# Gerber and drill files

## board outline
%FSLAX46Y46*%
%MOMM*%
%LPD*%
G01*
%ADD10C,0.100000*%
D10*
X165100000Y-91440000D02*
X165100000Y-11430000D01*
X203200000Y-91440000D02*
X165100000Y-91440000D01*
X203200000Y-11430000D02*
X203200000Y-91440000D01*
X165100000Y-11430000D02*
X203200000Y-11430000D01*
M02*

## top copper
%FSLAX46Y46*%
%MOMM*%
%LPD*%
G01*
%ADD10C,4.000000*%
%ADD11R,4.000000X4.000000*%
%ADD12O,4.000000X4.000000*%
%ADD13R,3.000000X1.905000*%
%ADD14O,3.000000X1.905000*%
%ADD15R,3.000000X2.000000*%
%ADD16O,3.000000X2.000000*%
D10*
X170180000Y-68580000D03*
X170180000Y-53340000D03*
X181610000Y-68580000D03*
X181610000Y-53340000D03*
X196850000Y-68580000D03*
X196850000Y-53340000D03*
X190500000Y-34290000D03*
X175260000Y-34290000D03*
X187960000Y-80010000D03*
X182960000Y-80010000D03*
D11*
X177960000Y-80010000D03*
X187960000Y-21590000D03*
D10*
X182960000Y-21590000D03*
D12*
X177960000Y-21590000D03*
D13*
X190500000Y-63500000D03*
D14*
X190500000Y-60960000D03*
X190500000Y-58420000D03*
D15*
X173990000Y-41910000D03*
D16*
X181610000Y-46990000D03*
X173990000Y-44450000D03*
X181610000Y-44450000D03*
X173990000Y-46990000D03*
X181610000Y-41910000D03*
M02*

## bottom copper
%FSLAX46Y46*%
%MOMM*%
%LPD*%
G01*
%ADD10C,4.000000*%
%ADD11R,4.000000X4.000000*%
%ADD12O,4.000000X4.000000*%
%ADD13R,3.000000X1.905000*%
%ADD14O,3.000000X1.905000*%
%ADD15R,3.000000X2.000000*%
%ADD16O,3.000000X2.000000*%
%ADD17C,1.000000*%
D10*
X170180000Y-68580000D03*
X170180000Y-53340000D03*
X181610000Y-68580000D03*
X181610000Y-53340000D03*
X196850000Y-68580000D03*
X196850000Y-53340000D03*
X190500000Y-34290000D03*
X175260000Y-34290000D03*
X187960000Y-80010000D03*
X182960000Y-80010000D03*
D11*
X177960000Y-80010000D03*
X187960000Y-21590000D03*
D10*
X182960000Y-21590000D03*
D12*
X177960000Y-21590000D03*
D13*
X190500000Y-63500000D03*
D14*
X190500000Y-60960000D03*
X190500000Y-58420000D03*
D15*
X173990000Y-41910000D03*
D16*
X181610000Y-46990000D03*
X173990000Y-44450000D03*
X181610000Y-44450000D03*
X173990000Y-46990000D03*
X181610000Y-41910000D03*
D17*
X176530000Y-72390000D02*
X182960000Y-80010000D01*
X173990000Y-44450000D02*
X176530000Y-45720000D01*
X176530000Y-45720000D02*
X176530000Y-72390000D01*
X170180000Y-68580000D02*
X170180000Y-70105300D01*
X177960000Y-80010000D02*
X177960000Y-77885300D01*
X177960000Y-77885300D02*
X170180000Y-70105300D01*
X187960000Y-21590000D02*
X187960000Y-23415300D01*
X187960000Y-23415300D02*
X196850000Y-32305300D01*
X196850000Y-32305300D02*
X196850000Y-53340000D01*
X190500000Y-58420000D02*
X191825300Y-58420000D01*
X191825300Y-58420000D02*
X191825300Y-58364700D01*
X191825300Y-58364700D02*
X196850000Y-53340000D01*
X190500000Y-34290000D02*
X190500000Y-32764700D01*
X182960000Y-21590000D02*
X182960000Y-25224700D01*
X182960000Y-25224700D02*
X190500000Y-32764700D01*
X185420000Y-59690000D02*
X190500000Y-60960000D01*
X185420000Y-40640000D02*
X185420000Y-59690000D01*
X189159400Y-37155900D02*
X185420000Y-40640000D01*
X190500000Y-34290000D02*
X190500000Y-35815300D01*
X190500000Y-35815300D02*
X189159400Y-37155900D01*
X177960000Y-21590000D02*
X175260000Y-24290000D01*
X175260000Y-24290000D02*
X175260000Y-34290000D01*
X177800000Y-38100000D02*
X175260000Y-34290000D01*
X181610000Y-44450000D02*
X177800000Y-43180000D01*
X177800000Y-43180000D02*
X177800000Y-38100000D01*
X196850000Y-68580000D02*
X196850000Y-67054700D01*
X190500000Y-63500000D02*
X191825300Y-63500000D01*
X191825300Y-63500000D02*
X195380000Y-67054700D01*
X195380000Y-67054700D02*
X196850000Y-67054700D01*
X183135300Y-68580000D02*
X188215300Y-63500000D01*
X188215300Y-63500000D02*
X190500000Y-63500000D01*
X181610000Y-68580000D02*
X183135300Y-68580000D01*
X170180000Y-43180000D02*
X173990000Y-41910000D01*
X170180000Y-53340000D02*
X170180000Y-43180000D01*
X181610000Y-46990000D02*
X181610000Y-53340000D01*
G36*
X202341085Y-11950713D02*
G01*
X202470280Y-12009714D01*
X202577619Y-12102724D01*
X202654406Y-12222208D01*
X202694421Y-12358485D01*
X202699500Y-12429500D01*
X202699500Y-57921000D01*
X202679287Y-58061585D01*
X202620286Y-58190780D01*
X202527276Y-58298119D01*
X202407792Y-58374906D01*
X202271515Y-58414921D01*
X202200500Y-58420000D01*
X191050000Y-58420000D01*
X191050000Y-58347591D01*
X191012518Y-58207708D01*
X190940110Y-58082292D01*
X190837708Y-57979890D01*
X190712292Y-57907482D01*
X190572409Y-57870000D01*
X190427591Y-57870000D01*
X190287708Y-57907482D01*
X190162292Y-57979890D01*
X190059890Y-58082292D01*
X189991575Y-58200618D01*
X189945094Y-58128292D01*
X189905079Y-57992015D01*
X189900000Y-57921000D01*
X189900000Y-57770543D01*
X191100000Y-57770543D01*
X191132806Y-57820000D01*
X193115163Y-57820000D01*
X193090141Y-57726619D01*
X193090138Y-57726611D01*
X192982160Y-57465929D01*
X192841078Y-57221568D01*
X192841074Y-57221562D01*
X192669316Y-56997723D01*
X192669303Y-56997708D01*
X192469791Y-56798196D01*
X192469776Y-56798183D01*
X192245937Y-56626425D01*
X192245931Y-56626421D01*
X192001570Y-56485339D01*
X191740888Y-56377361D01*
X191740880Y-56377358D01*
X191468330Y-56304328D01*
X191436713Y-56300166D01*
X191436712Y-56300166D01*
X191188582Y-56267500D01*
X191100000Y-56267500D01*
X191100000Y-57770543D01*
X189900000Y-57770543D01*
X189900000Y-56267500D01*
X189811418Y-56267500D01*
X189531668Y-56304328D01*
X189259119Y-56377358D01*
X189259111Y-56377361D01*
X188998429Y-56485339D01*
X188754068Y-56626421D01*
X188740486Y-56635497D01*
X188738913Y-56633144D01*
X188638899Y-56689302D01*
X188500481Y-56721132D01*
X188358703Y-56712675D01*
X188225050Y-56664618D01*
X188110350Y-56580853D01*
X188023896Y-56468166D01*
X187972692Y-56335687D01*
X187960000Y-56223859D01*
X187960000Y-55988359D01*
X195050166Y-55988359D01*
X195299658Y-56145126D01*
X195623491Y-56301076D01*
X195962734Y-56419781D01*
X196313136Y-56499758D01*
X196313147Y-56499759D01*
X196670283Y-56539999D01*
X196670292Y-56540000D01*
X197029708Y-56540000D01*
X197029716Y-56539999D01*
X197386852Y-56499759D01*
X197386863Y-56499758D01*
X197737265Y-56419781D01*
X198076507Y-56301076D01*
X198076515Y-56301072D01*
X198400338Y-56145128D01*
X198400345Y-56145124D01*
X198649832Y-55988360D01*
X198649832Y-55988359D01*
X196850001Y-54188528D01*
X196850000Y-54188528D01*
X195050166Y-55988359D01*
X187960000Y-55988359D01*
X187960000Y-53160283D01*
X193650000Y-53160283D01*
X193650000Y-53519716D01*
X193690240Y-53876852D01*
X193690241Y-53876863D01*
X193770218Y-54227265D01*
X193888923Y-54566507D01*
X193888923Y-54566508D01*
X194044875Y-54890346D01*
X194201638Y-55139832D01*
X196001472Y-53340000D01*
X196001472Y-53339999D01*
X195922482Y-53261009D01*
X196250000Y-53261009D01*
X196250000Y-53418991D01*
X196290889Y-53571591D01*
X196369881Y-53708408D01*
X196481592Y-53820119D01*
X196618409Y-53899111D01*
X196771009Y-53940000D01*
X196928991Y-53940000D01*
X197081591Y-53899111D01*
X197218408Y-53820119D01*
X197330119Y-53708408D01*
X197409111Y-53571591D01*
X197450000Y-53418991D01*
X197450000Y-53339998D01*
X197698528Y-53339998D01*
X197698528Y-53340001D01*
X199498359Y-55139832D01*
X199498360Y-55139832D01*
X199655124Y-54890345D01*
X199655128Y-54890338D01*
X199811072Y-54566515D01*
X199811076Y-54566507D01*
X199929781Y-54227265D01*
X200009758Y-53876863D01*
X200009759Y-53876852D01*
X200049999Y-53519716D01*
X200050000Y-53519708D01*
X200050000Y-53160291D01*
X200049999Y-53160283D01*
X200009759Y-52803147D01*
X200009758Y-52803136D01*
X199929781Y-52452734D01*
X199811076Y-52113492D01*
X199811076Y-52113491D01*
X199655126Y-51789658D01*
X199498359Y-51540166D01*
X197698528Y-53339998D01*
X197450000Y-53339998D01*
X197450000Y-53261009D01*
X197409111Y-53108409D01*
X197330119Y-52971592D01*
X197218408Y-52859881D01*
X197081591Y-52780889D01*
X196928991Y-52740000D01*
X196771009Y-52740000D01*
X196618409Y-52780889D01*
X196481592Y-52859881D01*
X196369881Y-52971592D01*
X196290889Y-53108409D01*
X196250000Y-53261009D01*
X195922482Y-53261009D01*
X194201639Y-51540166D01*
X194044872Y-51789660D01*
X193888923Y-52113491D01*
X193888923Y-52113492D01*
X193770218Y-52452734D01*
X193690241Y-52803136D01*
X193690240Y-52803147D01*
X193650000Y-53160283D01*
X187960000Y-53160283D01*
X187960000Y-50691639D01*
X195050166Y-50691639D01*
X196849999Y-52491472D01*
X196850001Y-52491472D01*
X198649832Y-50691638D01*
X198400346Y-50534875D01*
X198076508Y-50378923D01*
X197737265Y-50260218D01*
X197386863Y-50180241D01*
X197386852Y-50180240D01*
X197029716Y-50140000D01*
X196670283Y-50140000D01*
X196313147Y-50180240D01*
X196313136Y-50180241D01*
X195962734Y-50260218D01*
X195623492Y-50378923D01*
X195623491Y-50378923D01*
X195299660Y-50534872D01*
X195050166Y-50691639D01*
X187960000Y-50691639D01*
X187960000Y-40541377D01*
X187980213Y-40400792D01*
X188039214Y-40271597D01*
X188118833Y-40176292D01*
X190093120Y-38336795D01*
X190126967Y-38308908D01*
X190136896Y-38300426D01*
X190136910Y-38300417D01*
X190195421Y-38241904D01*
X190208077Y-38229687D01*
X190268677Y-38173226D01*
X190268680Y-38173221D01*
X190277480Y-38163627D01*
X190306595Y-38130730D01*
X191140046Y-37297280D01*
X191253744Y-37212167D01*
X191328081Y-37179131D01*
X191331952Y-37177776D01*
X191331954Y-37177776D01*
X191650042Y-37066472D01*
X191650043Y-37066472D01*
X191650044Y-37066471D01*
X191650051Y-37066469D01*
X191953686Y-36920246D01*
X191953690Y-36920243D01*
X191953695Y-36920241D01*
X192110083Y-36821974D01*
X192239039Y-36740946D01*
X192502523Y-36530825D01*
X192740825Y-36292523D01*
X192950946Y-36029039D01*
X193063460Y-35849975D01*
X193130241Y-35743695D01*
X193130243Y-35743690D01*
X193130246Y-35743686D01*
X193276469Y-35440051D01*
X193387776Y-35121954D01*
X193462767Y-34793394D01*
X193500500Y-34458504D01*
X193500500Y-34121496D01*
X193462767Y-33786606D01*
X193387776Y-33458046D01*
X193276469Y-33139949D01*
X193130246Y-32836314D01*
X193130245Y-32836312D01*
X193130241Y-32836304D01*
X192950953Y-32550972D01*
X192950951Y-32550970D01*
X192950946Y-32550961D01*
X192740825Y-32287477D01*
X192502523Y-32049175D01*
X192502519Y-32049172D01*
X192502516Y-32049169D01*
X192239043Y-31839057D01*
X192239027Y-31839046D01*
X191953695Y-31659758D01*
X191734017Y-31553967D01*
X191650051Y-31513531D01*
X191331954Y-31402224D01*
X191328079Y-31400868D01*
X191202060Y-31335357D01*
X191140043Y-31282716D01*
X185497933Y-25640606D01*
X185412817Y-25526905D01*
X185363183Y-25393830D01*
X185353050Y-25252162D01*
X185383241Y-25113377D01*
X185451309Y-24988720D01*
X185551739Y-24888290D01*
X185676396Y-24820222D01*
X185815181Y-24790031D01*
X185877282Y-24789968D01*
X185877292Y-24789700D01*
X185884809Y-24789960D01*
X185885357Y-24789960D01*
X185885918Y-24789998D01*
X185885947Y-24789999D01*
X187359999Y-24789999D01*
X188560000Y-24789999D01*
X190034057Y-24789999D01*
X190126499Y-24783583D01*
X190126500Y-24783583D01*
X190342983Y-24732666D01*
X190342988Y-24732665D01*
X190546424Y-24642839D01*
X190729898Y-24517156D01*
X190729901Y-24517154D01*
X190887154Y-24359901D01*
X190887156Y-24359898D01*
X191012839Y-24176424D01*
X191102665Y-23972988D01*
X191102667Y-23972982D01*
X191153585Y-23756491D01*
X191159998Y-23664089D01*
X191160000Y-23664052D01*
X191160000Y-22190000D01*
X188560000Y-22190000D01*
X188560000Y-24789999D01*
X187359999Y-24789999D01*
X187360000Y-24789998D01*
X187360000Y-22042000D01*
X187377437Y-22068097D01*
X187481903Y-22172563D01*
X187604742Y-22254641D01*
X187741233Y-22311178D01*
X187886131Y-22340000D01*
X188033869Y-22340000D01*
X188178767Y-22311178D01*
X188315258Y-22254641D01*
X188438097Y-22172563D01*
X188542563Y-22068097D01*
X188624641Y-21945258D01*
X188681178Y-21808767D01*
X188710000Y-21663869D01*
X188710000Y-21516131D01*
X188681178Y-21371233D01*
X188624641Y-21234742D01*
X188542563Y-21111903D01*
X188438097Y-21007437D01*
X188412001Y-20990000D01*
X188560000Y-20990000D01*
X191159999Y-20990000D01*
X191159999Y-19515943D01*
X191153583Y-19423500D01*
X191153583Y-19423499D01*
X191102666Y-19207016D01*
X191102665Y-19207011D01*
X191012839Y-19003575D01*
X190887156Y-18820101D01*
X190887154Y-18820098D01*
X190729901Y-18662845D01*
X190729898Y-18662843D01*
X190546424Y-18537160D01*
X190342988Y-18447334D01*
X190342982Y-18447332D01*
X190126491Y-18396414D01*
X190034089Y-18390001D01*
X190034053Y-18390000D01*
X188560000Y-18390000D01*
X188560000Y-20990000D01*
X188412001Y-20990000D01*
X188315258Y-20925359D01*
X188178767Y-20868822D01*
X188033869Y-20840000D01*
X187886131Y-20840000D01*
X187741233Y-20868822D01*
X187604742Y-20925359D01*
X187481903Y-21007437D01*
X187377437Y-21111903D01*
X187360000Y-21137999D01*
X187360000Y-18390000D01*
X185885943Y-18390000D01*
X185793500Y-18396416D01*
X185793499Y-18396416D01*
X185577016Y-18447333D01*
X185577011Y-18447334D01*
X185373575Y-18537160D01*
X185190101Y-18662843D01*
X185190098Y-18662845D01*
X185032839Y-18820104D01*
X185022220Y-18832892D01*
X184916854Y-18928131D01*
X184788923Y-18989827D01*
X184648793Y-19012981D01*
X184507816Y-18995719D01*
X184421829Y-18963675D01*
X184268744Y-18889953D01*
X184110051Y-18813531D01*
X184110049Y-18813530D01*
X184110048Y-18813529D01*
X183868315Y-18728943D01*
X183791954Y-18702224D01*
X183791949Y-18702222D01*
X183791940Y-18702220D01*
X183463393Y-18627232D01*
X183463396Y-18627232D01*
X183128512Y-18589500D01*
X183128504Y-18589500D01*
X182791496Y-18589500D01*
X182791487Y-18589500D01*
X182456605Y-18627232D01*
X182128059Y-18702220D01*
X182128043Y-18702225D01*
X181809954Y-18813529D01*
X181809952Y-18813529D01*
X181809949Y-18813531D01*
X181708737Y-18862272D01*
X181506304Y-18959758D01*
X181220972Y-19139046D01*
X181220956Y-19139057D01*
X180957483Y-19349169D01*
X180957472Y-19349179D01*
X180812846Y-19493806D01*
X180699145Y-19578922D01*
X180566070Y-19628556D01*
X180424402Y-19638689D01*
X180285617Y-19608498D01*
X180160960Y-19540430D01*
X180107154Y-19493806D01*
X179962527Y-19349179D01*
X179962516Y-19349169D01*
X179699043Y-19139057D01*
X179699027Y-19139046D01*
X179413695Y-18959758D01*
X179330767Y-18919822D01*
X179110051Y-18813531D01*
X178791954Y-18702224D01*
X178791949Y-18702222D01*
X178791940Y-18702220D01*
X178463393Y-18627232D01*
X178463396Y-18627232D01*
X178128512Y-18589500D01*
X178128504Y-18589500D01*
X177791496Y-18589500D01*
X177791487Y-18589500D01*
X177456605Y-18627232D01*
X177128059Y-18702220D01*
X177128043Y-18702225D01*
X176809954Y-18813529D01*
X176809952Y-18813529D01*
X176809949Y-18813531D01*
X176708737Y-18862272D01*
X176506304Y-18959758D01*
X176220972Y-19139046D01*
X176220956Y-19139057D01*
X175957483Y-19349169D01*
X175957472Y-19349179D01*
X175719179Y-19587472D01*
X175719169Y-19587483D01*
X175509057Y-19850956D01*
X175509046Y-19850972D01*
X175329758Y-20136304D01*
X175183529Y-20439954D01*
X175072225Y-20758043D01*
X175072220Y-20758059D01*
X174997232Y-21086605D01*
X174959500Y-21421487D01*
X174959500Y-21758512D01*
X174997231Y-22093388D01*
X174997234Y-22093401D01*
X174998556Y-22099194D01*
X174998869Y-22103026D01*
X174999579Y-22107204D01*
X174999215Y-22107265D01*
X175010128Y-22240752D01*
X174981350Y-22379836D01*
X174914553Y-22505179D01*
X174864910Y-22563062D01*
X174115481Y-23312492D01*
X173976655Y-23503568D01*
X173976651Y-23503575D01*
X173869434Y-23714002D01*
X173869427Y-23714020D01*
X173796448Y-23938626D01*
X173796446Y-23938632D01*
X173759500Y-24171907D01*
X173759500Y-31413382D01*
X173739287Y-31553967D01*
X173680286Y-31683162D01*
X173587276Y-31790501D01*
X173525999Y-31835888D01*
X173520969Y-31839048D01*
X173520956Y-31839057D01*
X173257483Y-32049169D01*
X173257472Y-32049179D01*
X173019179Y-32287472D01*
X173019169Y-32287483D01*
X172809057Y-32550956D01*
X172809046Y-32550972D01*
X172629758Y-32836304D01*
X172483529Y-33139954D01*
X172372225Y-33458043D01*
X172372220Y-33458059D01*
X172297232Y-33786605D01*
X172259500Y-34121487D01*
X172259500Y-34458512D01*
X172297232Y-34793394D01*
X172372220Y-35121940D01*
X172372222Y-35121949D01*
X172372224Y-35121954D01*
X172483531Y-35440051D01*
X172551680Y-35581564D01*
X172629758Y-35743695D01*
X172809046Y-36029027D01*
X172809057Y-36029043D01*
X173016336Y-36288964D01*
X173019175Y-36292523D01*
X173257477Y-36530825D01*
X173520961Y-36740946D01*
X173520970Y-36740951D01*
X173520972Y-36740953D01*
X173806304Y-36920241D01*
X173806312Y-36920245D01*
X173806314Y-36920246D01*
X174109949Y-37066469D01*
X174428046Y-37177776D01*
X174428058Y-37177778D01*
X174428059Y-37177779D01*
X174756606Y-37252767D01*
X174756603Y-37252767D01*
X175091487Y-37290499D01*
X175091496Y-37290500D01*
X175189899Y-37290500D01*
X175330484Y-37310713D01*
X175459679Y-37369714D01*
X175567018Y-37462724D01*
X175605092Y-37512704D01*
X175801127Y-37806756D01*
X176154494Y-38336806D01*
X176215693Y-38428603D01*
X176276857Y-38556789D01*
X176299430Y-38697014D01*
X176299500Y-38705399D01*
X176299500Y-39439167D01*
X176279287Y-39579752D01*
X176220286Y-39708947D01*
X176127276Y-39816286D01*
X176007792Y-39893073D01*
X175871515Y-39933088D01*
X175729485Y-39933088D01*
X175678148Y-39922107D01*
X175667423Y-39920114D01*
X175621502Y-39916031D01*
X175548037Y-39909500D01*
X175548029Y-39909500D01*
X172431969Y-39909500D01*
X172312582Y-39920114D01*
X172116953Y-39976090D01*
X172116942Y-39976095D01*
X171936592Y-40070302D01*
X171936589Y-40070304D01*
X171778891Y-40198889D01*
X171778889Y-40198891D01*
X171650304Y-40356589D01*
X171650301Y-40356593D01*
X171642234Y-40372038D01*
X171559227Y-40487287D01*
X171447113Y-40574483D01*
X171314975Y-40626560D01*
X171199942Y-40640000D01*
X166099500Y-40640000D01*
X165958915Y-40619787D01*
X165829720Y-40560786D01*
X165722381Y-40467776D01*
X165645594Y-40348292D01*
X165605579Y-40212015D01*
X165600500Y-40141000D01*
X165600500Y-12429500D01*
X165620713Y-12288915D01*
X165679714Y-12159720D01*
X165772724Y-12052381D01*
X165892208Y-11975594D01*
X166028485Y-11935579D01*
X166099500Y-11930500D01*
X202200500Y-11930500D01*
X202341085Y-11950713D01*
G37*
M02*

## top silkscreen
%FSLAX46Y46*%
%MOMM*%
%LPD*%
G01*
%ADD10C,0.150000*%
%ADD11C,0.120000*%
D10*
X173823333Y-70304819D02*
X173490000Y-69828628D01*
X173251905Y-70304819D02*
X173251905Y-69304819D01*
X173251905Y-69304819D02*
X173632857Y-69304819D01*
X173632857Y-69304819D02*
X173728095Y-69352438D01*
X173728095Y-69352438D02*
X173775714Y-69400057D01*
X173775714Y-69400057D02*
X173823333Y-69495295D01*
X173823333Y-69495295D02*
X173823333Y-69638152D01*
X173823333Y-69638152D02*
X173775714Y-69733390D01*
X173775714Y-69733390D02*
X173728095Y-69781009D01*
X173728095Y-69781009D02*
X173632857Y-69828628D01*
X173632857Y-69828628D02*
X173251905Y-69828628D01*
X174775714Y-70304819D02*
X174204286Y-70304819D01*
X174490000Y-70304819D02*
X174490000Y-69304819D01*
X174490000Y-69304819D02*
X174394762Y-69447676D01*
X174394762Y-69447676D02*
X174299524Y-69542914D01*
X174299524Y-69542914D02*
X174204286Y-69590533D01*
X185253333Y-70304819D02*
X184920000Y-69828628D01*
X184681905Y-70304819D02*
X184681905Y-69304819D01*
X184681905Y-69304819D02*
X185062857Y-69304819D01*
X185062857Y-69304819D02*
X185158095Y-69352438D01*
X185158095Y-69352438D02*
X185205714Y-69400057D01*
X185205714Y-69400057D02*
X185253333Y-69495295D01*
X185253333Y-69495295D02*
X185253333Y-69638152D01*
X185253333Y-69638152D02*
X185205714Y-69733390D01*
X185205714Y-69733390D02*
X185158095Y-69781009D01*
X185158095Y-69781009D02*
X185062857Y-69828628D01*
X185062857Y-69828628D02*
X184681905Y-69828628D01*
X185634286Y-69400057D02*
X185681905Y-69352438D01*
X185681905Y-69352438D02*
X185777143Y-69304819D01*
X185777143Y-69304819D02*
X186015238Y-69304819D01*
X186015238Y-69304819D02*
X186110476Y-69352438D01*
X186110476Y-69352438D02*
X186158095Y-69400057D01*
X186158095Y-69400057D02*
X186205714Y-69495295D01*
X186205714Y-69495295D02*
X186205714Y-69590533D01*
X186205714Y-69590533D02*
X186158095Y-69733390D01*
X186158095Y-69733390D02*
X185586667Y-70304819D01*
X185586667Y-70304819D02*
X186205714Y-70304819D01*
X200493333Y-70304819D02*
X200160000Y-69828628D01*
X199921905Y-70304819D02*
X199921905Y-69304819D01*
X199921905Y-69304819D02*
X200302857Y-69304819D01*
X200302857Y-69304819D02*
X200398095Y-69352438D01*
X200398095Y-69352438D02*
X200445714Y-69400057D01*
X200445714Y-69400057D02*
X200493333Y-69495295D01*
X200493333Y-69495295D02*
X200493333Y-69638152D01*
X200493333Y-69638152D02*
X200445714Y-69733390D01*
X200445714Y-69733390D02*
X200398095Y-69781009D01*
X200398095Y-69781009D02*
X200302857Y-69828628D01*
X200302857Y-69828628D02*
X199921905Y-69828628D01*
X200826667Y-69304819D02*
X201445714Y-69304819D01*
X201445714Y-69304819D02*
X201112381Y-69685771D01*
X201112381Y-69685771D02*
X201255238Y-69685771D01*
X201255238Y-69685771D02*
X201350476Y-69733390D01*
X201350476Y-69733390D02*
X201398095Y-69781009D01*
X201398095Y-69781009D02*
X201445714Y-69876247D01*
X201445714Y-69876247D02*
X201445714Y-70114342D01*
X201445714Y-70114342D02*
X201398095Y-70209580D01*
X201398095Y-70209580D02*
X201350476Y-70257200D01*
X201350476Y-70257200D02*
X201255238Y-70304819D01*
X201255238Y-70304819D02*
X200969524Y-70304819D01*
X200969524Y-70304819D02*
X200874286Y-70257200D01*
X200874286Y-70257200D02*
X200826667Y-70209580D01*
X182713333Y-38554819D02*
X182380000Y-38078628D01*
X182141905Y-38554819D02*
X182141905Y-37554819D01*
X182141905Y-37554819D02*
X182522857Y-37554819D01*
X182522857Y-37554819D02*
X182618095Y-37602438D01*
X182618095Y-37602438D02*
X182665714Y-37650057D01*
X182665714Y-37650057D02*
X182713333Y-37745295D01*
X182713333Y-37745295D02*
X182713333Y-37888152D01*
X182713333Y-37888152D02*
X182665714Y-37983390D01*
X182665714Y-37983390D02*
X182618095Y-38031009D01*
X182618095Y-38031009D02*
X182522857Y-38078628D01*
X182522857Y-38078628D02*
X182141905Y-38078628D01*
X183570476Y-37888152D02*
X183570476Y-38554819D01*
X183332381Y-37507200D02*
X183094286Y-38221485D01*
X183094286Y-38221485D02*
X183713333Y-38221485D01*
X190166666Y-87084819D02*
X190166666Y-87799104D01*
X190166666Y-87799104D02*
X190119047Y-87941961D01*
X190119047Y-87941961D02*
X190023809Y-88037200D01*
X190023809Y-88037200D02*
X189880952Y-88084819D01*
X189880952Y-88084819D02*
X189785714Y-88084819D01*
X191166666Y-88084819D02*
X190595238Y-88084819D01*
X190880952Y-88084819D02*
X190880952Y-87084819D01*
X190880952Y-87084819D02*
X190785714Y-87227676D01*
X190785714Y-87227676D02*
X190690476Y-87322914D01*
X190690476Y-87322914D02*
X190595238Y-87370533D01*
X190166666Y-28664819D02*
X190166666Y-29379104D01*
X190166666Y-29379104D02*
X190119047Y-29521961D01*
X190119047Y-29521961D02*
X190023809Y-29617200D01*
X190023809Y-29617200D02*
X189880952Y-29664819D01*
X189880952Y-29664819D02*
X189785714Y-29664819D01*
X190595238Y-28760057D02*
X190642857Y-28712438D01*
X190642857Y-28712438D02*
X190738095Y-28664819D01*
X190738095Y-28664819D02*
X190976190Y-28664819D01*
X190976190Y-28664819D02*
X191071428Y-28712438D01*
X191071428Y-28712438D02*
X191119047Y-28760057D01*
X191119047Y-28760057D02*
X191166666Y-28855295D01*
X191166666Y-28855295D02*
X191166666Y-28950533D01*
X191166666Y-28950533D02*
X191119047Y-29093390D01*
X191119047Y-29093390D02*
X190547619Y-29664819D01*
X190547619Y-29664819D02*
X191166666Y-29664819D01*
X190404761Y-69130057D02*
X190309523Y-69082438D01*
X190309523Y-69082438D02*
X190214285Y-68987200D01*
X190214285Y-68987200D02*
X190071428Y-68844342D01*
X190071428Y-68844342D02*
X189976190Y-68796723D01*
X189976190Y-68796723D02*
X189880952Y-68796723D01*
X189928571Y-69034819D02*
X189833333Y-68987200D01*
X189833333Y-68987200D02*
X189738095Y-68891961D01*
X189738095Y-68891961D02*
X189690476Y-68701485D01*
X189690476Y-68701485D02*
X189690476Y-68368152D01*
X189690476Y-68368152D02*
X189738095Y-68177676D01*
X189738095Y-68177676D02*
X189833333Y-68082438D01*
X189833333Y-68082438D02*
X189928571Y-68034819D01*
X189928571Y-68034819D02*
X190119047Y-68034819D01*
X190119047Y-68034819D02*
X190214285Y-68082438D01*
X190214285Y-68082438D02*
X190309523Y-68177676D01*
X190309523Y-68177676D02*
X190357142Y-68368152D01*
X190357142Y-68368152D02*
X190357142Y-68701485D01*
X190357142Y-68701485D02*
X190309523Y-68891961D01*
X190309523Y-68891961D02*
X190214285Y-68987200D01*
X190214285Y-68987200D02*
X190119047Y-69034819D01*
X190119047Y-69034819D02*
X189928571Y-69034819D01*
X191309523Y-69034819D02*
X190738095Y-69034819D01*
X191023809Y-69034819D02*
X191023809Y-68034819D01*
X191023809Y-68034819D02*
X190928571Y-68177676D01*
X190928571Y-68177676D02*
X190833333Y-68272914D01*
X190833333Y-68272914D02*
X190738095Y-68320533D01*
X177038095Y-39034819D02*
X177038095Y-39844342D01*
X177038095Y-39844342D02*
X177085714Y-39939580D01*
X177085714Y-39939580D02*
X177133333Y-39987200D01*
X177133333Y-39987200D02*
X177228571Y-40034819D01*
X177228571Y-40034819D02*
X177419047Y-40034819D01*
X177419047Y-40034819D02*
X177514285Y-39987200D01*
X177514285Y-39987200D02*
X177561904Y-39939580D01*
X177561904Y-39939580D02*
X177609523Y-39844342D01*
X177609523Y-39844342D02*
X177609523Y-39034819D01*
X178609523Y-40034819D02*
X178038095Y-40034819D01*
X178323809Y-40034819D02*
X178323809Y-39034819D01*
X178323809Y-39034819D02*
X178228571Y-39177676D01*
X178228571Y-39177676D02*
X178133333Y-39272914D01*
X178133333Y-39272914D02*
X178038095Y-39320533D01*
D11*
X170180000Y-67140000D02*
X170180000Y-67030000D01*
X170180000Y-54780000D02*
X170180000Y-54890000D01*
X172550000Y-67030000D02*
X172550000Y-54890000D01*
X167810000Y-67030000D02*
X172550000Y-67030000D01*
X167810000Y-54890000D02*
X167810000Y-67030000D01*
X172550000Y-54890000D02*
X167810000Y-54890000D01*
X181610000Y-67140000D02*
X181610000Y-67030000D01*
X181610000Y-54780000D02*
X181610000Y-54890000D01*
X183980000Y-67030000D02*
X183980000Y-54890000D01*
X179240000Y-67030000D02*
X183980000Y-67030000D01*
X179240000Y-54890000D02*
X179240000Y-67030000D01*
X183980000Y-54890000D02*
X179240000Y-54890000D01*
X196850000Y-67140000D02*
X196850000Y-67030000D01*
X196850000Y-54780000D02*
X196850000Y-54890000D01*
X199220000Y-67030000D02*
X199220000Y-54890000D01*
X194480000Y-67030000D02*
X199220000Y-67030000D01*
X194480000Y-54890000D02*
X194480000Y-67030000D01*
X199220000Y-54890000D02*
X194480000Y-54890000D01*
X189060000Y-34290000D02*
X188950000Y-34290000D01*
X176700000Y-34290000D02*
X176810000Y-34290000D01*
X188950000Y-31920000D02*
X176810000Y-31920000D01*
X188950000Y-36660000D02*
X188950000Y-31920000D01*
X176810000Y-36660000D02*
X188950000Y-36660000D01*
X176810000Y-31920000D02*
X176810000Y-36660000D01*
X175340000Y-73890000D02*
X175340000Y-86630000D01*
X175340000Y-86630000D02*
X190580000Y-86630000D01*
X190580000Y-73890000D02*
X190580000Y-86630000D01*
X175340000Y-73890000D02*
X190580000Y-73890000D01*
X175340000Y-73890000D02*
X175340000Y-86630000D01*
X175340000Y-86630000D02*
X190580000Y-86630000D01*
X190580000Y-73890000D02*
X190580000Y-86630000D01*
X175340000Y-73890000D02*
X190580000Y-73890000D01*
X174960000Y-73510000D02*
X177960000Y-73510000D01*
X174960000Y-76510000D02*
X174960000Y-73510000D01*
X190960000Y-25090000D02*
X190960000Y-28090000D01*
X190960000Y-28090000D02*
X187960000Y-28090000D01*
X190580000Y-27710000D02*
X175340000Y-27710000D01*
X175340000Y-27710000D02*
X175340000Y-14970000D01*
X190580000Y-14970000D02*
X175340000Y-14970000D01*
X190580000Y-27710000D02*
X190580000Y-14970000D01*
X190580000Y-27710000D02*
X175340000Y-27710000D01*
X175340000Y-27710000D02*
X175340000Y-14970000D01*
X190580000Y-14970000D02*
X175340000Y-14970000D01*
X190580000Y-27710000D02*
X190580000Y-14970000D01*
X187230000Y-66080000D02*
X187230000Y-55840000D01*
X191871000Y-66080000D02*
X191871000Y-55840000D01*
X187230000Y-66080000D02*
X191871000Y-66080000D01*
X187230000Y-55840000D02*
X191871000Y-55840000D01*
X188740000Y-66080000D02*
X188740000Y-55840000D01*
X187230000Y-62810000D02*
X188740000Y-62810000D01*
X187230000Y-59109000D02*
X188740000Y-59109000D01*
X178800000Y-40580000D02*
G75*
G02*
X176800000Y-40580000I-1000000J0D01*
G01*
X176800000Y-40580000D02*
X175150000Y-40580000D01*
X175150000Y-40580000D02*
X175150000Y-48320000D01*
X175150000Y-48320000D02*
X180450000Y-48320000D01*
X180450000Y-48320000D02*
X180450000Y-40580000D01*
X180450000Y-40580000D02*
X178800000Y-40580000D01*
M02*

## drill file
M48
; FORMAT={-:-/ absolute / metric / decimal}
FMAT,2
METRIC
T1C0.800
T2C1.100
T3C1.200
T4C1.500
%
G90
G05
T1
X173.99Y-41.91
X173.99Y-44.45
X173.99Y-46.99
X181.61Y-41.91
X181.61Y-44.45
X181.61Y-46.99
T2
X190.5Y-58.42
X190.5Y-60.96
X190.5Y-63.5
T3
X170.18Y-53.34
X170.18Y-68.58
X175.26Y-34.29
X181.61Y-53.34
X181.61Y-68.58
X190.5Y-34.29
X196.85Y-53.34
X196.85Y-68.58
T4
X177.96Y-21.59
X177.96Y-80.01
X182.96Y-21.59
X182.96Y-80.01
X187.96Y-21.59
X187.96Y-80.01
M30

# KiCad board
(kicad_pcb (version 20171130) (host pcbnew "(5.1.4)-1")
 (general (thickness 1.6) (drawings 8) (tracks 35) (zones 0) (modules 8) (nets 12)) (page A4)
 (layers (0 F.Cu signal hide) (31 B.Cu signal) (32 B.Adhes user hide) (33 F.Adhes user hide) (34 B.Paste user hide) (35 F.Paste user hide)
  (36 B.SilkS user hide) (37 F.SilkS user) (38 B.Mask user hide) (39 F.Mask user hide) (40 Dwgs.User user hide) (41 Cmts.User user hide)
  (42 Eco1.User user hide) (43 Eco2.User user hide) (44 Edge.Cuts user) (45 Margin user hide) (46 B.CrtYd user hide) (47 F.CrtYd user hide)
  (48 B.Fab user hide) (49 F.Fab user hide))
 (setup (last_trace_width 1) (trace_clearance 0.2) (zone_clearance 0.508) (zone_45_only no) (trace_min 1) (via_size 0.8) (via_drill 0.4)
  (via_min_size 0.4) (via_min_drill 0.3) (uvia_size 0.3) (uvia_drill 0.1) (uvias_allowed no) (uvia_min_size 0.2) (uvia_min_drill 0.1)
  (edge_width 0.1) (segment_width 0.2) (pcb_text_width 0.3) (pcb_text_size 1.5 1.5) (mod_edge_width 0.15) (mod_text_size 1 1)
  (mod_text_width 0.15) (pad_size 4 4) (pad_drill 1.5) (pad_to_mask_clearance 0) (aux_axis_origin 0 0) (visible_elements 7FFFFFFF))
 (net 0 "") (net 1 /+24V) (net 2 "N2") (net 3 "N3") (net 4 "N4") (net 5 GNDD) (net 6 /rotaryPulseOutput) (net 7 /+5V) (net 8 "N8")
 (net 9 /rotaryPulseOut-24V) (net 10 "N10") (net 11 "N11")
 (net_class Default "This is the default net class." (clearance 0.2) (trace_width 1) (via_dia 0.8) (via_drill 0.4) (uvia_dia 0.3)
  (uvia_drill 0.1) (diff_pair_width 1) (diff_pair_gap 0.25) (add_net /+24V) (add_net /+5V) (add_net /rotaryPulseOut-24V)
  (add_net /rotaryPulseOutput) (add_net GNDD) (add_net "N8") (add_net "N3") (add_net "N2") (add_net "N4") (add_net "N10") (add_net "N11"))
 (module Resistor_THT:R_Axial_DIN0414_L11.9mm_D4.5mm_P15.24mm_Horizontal (layer F.Cu) (at 170.18 53.34 270)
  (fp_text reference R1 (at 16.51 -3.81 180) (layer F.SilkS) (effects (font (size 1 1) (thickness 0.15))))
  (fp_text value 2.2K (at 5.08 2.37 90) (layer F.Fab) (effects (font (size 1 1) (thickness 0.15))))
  (fp_line (start 13.8 0) (end 13.69 0) (layer F.SilkS) (width 0.12))
  (fp_line (start 1.44 0) (end 1.55 0) (layer F.SilkS) (width 0.12))
  (fp_line (start 13.69 -2.37) (end 1.55 -2.37) (layer F.SilkS) (width 0.12))
  (fp_line (start 13.69 2.37) (end 13.69 -2.37) (layer F.SilkS) (width 0.12))
  (fp_line (start 1.55 2.37) (end 13.69 2.37) (layer F.SilkS) (width 0.12))
  (fp_line (start 1.55 -2.37) (end 1.55 2.37) (layer F.SilkS) (width 0.12))
  (pad 2 thru_hole circle (at 15.24 0 270) (size 4 4) (drill 1.2) (layers *.Cu *.Mask) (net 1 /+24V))
  (pad 1 thru_hole circle (at 0 0 270) (size 4 4) (drill 1.2) (layers *.Cu *.Mask) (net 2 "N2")))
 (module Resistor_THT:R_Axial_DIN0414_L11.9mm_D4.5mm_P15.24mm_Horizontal (layer F.Cu) (at 181.61 53.34 270)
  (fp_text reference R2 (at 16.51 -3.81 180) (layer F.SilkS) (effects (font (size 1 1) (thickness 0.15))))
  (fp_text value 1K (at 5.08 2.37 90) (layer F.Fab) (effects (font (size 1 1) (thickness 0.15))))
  (fp_line (start 13.8 0) (end 13.69 0) (layer F.SilkS) (width 0.12))
  (fp_line (start 1.44 0) (end 1.55 0) (layer F.SilkS) (width 0.12))
  (fp_line (start 13.69 -2.37) (end 1.55 -2.37) (layer F.SilkS) (width 0.12))
  (fp_line (start 13.69 2.37) (end 13.69 -2.37) (layer F.SilkS) (width 0.12))
  (fp_line (start 1.55 2.37) (end 13.69 2.37) (layer F.SilkS) (width 0.12))
  (fp_line (start 1.55 -2.37) (end 1.55 2.37) (layer F.SilkS) (width 0.12))
  (pad 2 thru_hole circle (at 15.24 0 270) (size 4 4) (drill 1.2) (layers *.Cu *.Mask) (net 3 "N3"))
  (pad 1 thru_hole circle (at 0 0 270) (size 4 4) (drill 1.2) (layers *.Cu *.Mask) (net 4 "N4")))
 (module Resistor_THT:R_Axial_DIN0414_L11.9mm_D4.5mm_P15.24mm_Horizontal (layer F.Cu) (at 196.85 53.34 270)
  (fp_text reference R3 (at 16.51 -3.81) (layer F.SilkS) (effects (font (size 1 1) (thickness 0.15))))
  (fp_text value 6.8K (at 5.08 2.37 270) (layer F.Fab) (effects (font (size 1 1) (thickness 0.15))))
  (fp_line (start 13.8 0) (end 13.69 0) (layer F.SilkS) (width 0.12))
  (fp_line (start 1.44 0) (end 1.55 0) (layer F.SilkS) (width 0.12))
  (fp_line (start 13.69 -2.37) (end 1.55 -2.37) (layer F.SilkS) (width 0.12))
  (fp_line (start 13.69 2.37) (end 13.69 -2.37) (layer F.SilkS) (width 0.12))
  (fp_line (start 1.55 2.37) (end 13.69 2.37) (layer F.SilkS) (width 0.12))
  (fp_line (start 1.55 -2.37) (end 1.55 2.37) (layer F.SilkS) (width 0.12))
  (pad 2 thru_hole circle (at 15.24 0 270) (size 4 4) (drill 1.2) (layers *.Cu *.Mask) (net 3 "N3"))
  (pad 1 thru_hole circle (at 0 0 270) (size 4 4) (drill 1.2) (layers *.Cu *.Mask) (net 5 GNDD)))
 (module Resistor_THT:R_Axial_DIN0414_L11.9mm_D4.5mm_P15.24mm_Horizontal (layer F.Cu) (at 175.26 34.29)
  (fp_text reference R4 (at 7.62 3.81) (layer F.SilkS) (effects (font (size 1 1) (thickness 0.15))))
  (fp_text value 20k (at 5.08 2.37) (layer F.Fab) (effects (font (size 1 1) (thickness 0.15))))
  (fp_line (start 13.8 0) (end 13.69 0) (layer F.SilkS) (width 0.12))
  (fp_line (start 1.44 0) (end 1.55 0) (layer F.SilkS) (width 0.12))
  (fp_line (start 13.69 -2.37) (end 1.55 -2.37) (layer F.SilkS) (width 0.12))
  (fp_line (start 13.69 2.37) (end 13.69 -2.37) (layer F.SilkS) (width 0.12))
  (fp_line (start 1.55 2.37) (end 13.69 2.37) (layer F.SilkS) (width 0.12))
  (fp_line (start 1.55 -2.37) (end 1.55 2.37) (layer F.SilkS) (width 0.12))
  (pad 2 thru_hole circle (at 15.24 0) (size 4 4) (drill 1.2) (layers *.Cu *.Mask) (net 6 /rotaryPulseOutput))
  (pad 1 thru_hole circle (at 0 0) (size 4 4) (drill 1.2) (layers *.Cu *.Mask) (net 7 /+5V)))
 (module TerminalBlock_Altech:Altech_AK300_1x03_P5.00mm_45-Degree (layer F.Cu) (at 177.96 80.01)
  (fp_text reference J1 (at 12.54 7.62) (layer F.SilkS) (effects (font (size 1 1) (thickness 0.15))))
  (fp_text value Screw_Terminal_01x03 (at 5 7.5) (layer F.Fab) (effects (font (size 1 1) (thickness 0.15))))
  (fp_line (start -2.62 -6.12) (end -2.62 6.62) (layer F.SilkS) (width 0.12))
  (fp_line (start -2.62 6.62) (end 12.62 6.62) (layer F.SilkS) (width 0.12))
  (fp_line (start 12.62 -6.12) (end 12.62 6.62) (layer F.SilkS) (width 0.12))
  (fp_line (start -2.62 -6.12) (end 12.62 -6.12) (layer F.SilkS) (width 0.12))
  (fp_line (start -2.62 -6.12) (end -2.62 6.62) (layer F.SilkS) (width 0.12))
  (fp_line (start -2.62 6.62) (end 12.62 6.62) (layer F.SilkS) (width 0.12))
  (fp_line (start 12.62 -6.12) (end 12.62 6.62) (layer F.SilkS) (width 0.12))
  (fp_line (start -2.62 -6.12) (end 12.62 -6.12) (layer F.SilkS) (width 0.12))
  (fp_line (start -3 -6.5) (end 0 -6.5) (layer F.SilkS) (width 0.12))
  (fp_line (start -3 -3.5) (end -3 -6.5) (layer F.SilkS) (width 0.12))
  (pad 3 thru_hole circle (at 10 0) (size 4 4) (drill 1.5) (layers *.Cu *.Mask) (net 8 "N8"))
  (pad 2 thru_hole circle (at 5 0) (size 4 4) (drill 1.5) (layers *.Cu *.Mask) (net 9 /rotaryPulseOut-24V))
  (pad 1 thru_hole rect (at 0 0) (size 4 4) (drill 1.5) (layers *.Cu *.Mask) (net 1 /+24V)))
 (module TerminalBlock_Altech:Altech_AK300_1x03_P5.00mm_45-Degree (layer F.Cu) (at 187.96 21.59 180)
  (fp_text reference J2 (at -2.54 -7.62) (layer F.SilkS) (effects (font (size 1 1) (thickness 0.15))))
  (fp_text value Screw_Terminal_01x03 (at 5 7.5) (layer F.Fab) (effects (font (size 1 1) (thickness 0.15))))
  (fp_line (start -3 -3.5) (end -3 -6.5) (layer F.SilkS) (width 0.12))
  (fp_line (start -3 -6.5) (end 0 -6.5) (layer F.SilkS) (width 0.12))
  (fp_line (start -2.62 -6.12) (end 12.62 -6.12) (layer F.SilkS) (width 0.12))
  (fp_line (start 12.62 -6.12) (end 12.62 6.62) (layer F.SilkS) (width 0.12))
  (fp_line (start -2.62 6.62) (end 12.62 6.62) (layer F.SilkS) (width 0.12))
  (fp_line (start -2.62 -6.12) (end -2.62 6.62) (layer F.SilkS) (width 0.12))
  (fp_line (start -2.62 -6.12) (end 12.62 -6.12) (layer F.SilkS) (width 0.12))
  (fp_line (start 12.62 -6.12) (end 12.62 6.62) (layer F.SilkS) (width 0.12))
  (fp_line (start -2.62 6.62) (end 12.62 6.62) (layer F.SilkS) (width 0.12))
  (fp_line (start -2.62 -6.12) (end -2.62 6.62) (layer F.SilkS) (width 0.12))
  (pad 1 thru_hole rect (at 0 0 180) (size 4 4) (drill 1.5) (layers *.Cu *.Mask) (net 5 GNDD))
  (pad 2 thru_hole circle (at 5 0 180) (size 4 4) (drill 1.5) (layers *.Cu *.Mask) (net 6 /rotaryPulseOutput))
  (pad 3 thru_hole oval (at 10 0 180) (size 4 4) (drill 1.5) (layers *.Cu *.Mask) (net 7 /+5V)))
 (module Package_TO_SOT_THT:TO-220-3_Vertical (layer F.Cu) (at 190.5 63.5 90)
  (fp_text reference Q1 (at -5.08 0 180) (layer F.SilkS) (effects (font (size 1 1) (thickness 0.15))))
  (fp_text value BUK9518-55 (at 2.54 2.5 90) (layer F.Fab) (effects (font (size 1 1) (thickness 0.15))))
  (fp_line (start -2.58 -3.27) (end 7.66 -3.27) (layer F.SilkS) (width 0.12))
  (fp_line (start -2.58 1.371) (end 7.66 1.371) (layer F.SilkS) (width 0.12))
  (fp_line (start -2.58 -3.27) (end -2.58 1.371) (layer F.SilkS) (width 0.12))
  (fp_line (start 7.66 -3.27) (end 7.66 1.371) (layer F.SilkS) (width 0.12))
  (fp_line (start -2.58 -1.76) (end 7.66 -1.76) (layer F.SilkS) (width 0.12))
  (fp_line (start 0.69 -3.27) (end 0.69 -1.76) (layer F.SilkS) (width 0.12))
  (fp_line (start 4.391 -3.27) (end 4.391 -1.76) (layer F.SilkS) (width 0.12))
  (pad 1 thru_hole rect (at 0 0 90) (size 1.905 3) (drill 1.1) (layers *.Cu *.Mask) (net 3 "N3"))
  (pad 2 thru_hole oval (at 2.54 0 90) (size 1.905 3) (drill 1.1) (layers *.Cu *.Mask) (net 6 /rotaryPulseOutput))
  (pad 3 thru_hole oval (at 5.08 0 90) (size 1.905 3) (drill 1.1) (layers *.Cu *.Mask) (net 5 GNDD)))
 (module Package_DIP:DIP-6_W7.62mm (layer F.Cu) (at 173.99 41.91)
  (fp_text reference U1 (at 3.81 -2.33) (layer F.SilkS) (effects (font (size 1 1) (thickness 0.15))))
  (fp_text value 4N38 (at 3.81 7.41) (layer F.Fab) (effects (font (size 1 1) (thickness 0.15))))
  (fp_arc (start 3.81 -1.33) (end 2.81 -1.33) (angle -180) (layer F.SilkS) (width 0.12))
  (fp_line (start 2.81 -1.33) (end 1.16 -1.33) (layer F.SilkS) (width 0.12))
  (fp_line (start 1.16 -1.33) (end 1.16 6.41) (layer F.SilkS) (width 0.12))
  (fp_line (start 1.16 6.41) (end 6.46 6.41) (layer F.SilkS) (width 0.12))
  (fp_line (start 6.46 6.41) (end 6.46 -1.33) (layer F.SilkS) (width 0.12))
  (fp_line (start 6.46 -1.33) (end 4.81 -1.33) (layer F.SilkS) (width 0.12))
  (pad 1 thru_hole rect (at 0 0) (size 3 2) (drill 0.8) (layers *.Cu *.Mask) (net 2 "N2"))
  (pad 4 thru_hole oval (at 7.62 5.08) (size 3 2) (drill 0.8) (layers *.Cu *.Mask) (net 4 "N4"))
  (pad 2 thru_hole oval (at 0 2.54) (size 3 2) (drill 0.8) (layers *.Cu *.Mask) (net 9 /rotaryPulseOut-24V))
  (pad 5 thru_hole oval (at 7.62 2.54) (size 3 2) (drill 0.8) (layers *.Cu *.Mask) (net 7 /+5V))
  (pad 3 thru_hole oval (at 0 5.08) (size 3 2) (drill 0.8) (layers *.Cu *.Mask) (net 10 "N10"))
  (pad 6 thru_hole oval (at 7.62 0) (size 3 2) (drill 0.8) (layers *.Cu *.Mask) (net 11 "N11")))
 (gr_line (start 165.1 91.44) (end 165.1 11.43) (layer Edge.Cuts) (width 0.1))
 (gr_line (start 203.2 91.44) (end 165.1 91.44) (layer Edge.Cuts) (width 0.1))
 (gr_line (start 203.2 11.43) (end 203.2 91.44) (layer Edge.Cuts) (width 0.1))
 (gr_line (start 165.1 11.43) (end 203.2 11.43) (layer Edge.Cuts) (width 0.1))
 (segment (start 176.53 72.39) (end 182.96 80.01) (width 1) (layer B.Cu) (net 9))
 (segment (start 173.99 44.45) (end 176.53 45.72) (width 1) (layer B.Cu) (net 9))
 (segment (start 176.53 45.72) (end 176.53 72.39) (width 1) (layer B.Cu) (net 9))
 (segment (start 170.18 68.58) (end 170.18 70.1053) (width 1) (layer B.Cu) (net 1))
 (segment (start 177.96 80.01) (end 177.96 77.8853) (width 1) (layer B.Cu) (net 1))
 (segment (start 177.96 77.8853) (end 170.18 70.1053) (width 1) (layer B.Cu) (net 1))
 (segment (start 187.96 21.59) (end 187.96 23.4153) (width 1) (layer B.Cu) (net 5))
 (segment (start 187.96 23.4153) (end 196.85 32.3053) (width 1) (layer B.Cu) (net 5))
 (segment (start 196.85 32.3053) (end 196.85 53.34) (width 1) (layer B.Cu) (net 5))
 (segment (start 190.5 58.42) (end 191.8253 58.42) (width 1) (layer B.Cu) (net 5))
 (segment (start 191.8253 58.42) (end 191.8253 58.3647) (width 1) (layer B.Cu) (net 5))
 (segment (start 191.8253 58.3647) (end 196.85 53.34) (width 1) (layer B.Cu) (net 5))
 (segment (start 190.5 34.29) (end 190.5 32.7647) (width 1) (layer B.Cu) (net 6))
 (segment (start 182.96 21.59) (end 182.96 25.2247) (width 1) (layer B.Cu) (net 6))
 (segment (start 182.96 25.2247) (end 190.5 32.7647) (width 1) (layer B.Cu) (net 6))
 (segment (start 185.42 59.69) (end 190.5 60.96) (width 1) (layer B.Cu) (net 6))
 (segment (start 185.42 40.64) (end 185.42 59.69) (width 1) (layer B.Cu) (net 6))
 (segment (start 189.1594 37.1559) (end 185.42 40.64) (width 1) (layer B.Cu) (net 6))
 (segment (start 190.5 34.29) (end 190.5 35.8153) (width 1) (layer B.Cu) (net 6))
 (segment (start 190.5 35.8153) (end 189.1594 37.1559) (width 1) (layer B.Cu) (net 6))
 (segment (start 177.96 21.59) (end 175.26 24.29) (width 1) (layer B.Cu) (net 7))
 (segment (start 175.26 24.29) (end 175.26 34.29) (width 1) (layer B.Cu) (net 7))
 (segment (start 177.8 38.1) (end 175.26 34.29) (width 1) (layer B.Cu) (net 7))
 (segment (start 181.61 44.45) (end 177.8 43.18) (width 1) (layer B.Cu) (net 7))
 (segment (start 177.8 43.18) (end 177.8 38.1) (width 1) (layer B.Cu) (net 7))
 (segment (start 196.85 68.58) (end 196.85 67.0547) (width 1) (layer B.Cu) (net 3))
 (segment (start 190.5 63.5) (end 191.8253 63.5) (width 1) (layer B.Cu) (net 3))
 (segment (start 191.8253 63.5) (end 195.38 67.0547) (width 1) (layer B.Cu) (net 3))
 (segment (start 195.38 67.0547) (end 196.85 67.0547) (width 1) (layer B.Cu) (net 3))
 (segment (start 183.1353 68.58) (end 188.2153 63.5) (width 1) (layer B.Cu) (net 3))
 (segment (start 188.2153 63.5) (end 190.5 63.5) (width 1) (layer B.Cu) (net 3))
 (segment (start 181.61 68.58) (end 183.1353 68.58) (width 1) (layer B.Cu) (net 3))
 (segment (start 170.18 43.18) (end 173.99 41.91) (width 1) (layer B.Cu) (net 2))
 (segment (start 170.18 53.34) (end 170.18 43.18) (width 1) (layer B.Cu) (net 2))
 (segment (start 181.61 46.99) (end 181.61 53.34) (width 1) (layer B.Cu) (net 4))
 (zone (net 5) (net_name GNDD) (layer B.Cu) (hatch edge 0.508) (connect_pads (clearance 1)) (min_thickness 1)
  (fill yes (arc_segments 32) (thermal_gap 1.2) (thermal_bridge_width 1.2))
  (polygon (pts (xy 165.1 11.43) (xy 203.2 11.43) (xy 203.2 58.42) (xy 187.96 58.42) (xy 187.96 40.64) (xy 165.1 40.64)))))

